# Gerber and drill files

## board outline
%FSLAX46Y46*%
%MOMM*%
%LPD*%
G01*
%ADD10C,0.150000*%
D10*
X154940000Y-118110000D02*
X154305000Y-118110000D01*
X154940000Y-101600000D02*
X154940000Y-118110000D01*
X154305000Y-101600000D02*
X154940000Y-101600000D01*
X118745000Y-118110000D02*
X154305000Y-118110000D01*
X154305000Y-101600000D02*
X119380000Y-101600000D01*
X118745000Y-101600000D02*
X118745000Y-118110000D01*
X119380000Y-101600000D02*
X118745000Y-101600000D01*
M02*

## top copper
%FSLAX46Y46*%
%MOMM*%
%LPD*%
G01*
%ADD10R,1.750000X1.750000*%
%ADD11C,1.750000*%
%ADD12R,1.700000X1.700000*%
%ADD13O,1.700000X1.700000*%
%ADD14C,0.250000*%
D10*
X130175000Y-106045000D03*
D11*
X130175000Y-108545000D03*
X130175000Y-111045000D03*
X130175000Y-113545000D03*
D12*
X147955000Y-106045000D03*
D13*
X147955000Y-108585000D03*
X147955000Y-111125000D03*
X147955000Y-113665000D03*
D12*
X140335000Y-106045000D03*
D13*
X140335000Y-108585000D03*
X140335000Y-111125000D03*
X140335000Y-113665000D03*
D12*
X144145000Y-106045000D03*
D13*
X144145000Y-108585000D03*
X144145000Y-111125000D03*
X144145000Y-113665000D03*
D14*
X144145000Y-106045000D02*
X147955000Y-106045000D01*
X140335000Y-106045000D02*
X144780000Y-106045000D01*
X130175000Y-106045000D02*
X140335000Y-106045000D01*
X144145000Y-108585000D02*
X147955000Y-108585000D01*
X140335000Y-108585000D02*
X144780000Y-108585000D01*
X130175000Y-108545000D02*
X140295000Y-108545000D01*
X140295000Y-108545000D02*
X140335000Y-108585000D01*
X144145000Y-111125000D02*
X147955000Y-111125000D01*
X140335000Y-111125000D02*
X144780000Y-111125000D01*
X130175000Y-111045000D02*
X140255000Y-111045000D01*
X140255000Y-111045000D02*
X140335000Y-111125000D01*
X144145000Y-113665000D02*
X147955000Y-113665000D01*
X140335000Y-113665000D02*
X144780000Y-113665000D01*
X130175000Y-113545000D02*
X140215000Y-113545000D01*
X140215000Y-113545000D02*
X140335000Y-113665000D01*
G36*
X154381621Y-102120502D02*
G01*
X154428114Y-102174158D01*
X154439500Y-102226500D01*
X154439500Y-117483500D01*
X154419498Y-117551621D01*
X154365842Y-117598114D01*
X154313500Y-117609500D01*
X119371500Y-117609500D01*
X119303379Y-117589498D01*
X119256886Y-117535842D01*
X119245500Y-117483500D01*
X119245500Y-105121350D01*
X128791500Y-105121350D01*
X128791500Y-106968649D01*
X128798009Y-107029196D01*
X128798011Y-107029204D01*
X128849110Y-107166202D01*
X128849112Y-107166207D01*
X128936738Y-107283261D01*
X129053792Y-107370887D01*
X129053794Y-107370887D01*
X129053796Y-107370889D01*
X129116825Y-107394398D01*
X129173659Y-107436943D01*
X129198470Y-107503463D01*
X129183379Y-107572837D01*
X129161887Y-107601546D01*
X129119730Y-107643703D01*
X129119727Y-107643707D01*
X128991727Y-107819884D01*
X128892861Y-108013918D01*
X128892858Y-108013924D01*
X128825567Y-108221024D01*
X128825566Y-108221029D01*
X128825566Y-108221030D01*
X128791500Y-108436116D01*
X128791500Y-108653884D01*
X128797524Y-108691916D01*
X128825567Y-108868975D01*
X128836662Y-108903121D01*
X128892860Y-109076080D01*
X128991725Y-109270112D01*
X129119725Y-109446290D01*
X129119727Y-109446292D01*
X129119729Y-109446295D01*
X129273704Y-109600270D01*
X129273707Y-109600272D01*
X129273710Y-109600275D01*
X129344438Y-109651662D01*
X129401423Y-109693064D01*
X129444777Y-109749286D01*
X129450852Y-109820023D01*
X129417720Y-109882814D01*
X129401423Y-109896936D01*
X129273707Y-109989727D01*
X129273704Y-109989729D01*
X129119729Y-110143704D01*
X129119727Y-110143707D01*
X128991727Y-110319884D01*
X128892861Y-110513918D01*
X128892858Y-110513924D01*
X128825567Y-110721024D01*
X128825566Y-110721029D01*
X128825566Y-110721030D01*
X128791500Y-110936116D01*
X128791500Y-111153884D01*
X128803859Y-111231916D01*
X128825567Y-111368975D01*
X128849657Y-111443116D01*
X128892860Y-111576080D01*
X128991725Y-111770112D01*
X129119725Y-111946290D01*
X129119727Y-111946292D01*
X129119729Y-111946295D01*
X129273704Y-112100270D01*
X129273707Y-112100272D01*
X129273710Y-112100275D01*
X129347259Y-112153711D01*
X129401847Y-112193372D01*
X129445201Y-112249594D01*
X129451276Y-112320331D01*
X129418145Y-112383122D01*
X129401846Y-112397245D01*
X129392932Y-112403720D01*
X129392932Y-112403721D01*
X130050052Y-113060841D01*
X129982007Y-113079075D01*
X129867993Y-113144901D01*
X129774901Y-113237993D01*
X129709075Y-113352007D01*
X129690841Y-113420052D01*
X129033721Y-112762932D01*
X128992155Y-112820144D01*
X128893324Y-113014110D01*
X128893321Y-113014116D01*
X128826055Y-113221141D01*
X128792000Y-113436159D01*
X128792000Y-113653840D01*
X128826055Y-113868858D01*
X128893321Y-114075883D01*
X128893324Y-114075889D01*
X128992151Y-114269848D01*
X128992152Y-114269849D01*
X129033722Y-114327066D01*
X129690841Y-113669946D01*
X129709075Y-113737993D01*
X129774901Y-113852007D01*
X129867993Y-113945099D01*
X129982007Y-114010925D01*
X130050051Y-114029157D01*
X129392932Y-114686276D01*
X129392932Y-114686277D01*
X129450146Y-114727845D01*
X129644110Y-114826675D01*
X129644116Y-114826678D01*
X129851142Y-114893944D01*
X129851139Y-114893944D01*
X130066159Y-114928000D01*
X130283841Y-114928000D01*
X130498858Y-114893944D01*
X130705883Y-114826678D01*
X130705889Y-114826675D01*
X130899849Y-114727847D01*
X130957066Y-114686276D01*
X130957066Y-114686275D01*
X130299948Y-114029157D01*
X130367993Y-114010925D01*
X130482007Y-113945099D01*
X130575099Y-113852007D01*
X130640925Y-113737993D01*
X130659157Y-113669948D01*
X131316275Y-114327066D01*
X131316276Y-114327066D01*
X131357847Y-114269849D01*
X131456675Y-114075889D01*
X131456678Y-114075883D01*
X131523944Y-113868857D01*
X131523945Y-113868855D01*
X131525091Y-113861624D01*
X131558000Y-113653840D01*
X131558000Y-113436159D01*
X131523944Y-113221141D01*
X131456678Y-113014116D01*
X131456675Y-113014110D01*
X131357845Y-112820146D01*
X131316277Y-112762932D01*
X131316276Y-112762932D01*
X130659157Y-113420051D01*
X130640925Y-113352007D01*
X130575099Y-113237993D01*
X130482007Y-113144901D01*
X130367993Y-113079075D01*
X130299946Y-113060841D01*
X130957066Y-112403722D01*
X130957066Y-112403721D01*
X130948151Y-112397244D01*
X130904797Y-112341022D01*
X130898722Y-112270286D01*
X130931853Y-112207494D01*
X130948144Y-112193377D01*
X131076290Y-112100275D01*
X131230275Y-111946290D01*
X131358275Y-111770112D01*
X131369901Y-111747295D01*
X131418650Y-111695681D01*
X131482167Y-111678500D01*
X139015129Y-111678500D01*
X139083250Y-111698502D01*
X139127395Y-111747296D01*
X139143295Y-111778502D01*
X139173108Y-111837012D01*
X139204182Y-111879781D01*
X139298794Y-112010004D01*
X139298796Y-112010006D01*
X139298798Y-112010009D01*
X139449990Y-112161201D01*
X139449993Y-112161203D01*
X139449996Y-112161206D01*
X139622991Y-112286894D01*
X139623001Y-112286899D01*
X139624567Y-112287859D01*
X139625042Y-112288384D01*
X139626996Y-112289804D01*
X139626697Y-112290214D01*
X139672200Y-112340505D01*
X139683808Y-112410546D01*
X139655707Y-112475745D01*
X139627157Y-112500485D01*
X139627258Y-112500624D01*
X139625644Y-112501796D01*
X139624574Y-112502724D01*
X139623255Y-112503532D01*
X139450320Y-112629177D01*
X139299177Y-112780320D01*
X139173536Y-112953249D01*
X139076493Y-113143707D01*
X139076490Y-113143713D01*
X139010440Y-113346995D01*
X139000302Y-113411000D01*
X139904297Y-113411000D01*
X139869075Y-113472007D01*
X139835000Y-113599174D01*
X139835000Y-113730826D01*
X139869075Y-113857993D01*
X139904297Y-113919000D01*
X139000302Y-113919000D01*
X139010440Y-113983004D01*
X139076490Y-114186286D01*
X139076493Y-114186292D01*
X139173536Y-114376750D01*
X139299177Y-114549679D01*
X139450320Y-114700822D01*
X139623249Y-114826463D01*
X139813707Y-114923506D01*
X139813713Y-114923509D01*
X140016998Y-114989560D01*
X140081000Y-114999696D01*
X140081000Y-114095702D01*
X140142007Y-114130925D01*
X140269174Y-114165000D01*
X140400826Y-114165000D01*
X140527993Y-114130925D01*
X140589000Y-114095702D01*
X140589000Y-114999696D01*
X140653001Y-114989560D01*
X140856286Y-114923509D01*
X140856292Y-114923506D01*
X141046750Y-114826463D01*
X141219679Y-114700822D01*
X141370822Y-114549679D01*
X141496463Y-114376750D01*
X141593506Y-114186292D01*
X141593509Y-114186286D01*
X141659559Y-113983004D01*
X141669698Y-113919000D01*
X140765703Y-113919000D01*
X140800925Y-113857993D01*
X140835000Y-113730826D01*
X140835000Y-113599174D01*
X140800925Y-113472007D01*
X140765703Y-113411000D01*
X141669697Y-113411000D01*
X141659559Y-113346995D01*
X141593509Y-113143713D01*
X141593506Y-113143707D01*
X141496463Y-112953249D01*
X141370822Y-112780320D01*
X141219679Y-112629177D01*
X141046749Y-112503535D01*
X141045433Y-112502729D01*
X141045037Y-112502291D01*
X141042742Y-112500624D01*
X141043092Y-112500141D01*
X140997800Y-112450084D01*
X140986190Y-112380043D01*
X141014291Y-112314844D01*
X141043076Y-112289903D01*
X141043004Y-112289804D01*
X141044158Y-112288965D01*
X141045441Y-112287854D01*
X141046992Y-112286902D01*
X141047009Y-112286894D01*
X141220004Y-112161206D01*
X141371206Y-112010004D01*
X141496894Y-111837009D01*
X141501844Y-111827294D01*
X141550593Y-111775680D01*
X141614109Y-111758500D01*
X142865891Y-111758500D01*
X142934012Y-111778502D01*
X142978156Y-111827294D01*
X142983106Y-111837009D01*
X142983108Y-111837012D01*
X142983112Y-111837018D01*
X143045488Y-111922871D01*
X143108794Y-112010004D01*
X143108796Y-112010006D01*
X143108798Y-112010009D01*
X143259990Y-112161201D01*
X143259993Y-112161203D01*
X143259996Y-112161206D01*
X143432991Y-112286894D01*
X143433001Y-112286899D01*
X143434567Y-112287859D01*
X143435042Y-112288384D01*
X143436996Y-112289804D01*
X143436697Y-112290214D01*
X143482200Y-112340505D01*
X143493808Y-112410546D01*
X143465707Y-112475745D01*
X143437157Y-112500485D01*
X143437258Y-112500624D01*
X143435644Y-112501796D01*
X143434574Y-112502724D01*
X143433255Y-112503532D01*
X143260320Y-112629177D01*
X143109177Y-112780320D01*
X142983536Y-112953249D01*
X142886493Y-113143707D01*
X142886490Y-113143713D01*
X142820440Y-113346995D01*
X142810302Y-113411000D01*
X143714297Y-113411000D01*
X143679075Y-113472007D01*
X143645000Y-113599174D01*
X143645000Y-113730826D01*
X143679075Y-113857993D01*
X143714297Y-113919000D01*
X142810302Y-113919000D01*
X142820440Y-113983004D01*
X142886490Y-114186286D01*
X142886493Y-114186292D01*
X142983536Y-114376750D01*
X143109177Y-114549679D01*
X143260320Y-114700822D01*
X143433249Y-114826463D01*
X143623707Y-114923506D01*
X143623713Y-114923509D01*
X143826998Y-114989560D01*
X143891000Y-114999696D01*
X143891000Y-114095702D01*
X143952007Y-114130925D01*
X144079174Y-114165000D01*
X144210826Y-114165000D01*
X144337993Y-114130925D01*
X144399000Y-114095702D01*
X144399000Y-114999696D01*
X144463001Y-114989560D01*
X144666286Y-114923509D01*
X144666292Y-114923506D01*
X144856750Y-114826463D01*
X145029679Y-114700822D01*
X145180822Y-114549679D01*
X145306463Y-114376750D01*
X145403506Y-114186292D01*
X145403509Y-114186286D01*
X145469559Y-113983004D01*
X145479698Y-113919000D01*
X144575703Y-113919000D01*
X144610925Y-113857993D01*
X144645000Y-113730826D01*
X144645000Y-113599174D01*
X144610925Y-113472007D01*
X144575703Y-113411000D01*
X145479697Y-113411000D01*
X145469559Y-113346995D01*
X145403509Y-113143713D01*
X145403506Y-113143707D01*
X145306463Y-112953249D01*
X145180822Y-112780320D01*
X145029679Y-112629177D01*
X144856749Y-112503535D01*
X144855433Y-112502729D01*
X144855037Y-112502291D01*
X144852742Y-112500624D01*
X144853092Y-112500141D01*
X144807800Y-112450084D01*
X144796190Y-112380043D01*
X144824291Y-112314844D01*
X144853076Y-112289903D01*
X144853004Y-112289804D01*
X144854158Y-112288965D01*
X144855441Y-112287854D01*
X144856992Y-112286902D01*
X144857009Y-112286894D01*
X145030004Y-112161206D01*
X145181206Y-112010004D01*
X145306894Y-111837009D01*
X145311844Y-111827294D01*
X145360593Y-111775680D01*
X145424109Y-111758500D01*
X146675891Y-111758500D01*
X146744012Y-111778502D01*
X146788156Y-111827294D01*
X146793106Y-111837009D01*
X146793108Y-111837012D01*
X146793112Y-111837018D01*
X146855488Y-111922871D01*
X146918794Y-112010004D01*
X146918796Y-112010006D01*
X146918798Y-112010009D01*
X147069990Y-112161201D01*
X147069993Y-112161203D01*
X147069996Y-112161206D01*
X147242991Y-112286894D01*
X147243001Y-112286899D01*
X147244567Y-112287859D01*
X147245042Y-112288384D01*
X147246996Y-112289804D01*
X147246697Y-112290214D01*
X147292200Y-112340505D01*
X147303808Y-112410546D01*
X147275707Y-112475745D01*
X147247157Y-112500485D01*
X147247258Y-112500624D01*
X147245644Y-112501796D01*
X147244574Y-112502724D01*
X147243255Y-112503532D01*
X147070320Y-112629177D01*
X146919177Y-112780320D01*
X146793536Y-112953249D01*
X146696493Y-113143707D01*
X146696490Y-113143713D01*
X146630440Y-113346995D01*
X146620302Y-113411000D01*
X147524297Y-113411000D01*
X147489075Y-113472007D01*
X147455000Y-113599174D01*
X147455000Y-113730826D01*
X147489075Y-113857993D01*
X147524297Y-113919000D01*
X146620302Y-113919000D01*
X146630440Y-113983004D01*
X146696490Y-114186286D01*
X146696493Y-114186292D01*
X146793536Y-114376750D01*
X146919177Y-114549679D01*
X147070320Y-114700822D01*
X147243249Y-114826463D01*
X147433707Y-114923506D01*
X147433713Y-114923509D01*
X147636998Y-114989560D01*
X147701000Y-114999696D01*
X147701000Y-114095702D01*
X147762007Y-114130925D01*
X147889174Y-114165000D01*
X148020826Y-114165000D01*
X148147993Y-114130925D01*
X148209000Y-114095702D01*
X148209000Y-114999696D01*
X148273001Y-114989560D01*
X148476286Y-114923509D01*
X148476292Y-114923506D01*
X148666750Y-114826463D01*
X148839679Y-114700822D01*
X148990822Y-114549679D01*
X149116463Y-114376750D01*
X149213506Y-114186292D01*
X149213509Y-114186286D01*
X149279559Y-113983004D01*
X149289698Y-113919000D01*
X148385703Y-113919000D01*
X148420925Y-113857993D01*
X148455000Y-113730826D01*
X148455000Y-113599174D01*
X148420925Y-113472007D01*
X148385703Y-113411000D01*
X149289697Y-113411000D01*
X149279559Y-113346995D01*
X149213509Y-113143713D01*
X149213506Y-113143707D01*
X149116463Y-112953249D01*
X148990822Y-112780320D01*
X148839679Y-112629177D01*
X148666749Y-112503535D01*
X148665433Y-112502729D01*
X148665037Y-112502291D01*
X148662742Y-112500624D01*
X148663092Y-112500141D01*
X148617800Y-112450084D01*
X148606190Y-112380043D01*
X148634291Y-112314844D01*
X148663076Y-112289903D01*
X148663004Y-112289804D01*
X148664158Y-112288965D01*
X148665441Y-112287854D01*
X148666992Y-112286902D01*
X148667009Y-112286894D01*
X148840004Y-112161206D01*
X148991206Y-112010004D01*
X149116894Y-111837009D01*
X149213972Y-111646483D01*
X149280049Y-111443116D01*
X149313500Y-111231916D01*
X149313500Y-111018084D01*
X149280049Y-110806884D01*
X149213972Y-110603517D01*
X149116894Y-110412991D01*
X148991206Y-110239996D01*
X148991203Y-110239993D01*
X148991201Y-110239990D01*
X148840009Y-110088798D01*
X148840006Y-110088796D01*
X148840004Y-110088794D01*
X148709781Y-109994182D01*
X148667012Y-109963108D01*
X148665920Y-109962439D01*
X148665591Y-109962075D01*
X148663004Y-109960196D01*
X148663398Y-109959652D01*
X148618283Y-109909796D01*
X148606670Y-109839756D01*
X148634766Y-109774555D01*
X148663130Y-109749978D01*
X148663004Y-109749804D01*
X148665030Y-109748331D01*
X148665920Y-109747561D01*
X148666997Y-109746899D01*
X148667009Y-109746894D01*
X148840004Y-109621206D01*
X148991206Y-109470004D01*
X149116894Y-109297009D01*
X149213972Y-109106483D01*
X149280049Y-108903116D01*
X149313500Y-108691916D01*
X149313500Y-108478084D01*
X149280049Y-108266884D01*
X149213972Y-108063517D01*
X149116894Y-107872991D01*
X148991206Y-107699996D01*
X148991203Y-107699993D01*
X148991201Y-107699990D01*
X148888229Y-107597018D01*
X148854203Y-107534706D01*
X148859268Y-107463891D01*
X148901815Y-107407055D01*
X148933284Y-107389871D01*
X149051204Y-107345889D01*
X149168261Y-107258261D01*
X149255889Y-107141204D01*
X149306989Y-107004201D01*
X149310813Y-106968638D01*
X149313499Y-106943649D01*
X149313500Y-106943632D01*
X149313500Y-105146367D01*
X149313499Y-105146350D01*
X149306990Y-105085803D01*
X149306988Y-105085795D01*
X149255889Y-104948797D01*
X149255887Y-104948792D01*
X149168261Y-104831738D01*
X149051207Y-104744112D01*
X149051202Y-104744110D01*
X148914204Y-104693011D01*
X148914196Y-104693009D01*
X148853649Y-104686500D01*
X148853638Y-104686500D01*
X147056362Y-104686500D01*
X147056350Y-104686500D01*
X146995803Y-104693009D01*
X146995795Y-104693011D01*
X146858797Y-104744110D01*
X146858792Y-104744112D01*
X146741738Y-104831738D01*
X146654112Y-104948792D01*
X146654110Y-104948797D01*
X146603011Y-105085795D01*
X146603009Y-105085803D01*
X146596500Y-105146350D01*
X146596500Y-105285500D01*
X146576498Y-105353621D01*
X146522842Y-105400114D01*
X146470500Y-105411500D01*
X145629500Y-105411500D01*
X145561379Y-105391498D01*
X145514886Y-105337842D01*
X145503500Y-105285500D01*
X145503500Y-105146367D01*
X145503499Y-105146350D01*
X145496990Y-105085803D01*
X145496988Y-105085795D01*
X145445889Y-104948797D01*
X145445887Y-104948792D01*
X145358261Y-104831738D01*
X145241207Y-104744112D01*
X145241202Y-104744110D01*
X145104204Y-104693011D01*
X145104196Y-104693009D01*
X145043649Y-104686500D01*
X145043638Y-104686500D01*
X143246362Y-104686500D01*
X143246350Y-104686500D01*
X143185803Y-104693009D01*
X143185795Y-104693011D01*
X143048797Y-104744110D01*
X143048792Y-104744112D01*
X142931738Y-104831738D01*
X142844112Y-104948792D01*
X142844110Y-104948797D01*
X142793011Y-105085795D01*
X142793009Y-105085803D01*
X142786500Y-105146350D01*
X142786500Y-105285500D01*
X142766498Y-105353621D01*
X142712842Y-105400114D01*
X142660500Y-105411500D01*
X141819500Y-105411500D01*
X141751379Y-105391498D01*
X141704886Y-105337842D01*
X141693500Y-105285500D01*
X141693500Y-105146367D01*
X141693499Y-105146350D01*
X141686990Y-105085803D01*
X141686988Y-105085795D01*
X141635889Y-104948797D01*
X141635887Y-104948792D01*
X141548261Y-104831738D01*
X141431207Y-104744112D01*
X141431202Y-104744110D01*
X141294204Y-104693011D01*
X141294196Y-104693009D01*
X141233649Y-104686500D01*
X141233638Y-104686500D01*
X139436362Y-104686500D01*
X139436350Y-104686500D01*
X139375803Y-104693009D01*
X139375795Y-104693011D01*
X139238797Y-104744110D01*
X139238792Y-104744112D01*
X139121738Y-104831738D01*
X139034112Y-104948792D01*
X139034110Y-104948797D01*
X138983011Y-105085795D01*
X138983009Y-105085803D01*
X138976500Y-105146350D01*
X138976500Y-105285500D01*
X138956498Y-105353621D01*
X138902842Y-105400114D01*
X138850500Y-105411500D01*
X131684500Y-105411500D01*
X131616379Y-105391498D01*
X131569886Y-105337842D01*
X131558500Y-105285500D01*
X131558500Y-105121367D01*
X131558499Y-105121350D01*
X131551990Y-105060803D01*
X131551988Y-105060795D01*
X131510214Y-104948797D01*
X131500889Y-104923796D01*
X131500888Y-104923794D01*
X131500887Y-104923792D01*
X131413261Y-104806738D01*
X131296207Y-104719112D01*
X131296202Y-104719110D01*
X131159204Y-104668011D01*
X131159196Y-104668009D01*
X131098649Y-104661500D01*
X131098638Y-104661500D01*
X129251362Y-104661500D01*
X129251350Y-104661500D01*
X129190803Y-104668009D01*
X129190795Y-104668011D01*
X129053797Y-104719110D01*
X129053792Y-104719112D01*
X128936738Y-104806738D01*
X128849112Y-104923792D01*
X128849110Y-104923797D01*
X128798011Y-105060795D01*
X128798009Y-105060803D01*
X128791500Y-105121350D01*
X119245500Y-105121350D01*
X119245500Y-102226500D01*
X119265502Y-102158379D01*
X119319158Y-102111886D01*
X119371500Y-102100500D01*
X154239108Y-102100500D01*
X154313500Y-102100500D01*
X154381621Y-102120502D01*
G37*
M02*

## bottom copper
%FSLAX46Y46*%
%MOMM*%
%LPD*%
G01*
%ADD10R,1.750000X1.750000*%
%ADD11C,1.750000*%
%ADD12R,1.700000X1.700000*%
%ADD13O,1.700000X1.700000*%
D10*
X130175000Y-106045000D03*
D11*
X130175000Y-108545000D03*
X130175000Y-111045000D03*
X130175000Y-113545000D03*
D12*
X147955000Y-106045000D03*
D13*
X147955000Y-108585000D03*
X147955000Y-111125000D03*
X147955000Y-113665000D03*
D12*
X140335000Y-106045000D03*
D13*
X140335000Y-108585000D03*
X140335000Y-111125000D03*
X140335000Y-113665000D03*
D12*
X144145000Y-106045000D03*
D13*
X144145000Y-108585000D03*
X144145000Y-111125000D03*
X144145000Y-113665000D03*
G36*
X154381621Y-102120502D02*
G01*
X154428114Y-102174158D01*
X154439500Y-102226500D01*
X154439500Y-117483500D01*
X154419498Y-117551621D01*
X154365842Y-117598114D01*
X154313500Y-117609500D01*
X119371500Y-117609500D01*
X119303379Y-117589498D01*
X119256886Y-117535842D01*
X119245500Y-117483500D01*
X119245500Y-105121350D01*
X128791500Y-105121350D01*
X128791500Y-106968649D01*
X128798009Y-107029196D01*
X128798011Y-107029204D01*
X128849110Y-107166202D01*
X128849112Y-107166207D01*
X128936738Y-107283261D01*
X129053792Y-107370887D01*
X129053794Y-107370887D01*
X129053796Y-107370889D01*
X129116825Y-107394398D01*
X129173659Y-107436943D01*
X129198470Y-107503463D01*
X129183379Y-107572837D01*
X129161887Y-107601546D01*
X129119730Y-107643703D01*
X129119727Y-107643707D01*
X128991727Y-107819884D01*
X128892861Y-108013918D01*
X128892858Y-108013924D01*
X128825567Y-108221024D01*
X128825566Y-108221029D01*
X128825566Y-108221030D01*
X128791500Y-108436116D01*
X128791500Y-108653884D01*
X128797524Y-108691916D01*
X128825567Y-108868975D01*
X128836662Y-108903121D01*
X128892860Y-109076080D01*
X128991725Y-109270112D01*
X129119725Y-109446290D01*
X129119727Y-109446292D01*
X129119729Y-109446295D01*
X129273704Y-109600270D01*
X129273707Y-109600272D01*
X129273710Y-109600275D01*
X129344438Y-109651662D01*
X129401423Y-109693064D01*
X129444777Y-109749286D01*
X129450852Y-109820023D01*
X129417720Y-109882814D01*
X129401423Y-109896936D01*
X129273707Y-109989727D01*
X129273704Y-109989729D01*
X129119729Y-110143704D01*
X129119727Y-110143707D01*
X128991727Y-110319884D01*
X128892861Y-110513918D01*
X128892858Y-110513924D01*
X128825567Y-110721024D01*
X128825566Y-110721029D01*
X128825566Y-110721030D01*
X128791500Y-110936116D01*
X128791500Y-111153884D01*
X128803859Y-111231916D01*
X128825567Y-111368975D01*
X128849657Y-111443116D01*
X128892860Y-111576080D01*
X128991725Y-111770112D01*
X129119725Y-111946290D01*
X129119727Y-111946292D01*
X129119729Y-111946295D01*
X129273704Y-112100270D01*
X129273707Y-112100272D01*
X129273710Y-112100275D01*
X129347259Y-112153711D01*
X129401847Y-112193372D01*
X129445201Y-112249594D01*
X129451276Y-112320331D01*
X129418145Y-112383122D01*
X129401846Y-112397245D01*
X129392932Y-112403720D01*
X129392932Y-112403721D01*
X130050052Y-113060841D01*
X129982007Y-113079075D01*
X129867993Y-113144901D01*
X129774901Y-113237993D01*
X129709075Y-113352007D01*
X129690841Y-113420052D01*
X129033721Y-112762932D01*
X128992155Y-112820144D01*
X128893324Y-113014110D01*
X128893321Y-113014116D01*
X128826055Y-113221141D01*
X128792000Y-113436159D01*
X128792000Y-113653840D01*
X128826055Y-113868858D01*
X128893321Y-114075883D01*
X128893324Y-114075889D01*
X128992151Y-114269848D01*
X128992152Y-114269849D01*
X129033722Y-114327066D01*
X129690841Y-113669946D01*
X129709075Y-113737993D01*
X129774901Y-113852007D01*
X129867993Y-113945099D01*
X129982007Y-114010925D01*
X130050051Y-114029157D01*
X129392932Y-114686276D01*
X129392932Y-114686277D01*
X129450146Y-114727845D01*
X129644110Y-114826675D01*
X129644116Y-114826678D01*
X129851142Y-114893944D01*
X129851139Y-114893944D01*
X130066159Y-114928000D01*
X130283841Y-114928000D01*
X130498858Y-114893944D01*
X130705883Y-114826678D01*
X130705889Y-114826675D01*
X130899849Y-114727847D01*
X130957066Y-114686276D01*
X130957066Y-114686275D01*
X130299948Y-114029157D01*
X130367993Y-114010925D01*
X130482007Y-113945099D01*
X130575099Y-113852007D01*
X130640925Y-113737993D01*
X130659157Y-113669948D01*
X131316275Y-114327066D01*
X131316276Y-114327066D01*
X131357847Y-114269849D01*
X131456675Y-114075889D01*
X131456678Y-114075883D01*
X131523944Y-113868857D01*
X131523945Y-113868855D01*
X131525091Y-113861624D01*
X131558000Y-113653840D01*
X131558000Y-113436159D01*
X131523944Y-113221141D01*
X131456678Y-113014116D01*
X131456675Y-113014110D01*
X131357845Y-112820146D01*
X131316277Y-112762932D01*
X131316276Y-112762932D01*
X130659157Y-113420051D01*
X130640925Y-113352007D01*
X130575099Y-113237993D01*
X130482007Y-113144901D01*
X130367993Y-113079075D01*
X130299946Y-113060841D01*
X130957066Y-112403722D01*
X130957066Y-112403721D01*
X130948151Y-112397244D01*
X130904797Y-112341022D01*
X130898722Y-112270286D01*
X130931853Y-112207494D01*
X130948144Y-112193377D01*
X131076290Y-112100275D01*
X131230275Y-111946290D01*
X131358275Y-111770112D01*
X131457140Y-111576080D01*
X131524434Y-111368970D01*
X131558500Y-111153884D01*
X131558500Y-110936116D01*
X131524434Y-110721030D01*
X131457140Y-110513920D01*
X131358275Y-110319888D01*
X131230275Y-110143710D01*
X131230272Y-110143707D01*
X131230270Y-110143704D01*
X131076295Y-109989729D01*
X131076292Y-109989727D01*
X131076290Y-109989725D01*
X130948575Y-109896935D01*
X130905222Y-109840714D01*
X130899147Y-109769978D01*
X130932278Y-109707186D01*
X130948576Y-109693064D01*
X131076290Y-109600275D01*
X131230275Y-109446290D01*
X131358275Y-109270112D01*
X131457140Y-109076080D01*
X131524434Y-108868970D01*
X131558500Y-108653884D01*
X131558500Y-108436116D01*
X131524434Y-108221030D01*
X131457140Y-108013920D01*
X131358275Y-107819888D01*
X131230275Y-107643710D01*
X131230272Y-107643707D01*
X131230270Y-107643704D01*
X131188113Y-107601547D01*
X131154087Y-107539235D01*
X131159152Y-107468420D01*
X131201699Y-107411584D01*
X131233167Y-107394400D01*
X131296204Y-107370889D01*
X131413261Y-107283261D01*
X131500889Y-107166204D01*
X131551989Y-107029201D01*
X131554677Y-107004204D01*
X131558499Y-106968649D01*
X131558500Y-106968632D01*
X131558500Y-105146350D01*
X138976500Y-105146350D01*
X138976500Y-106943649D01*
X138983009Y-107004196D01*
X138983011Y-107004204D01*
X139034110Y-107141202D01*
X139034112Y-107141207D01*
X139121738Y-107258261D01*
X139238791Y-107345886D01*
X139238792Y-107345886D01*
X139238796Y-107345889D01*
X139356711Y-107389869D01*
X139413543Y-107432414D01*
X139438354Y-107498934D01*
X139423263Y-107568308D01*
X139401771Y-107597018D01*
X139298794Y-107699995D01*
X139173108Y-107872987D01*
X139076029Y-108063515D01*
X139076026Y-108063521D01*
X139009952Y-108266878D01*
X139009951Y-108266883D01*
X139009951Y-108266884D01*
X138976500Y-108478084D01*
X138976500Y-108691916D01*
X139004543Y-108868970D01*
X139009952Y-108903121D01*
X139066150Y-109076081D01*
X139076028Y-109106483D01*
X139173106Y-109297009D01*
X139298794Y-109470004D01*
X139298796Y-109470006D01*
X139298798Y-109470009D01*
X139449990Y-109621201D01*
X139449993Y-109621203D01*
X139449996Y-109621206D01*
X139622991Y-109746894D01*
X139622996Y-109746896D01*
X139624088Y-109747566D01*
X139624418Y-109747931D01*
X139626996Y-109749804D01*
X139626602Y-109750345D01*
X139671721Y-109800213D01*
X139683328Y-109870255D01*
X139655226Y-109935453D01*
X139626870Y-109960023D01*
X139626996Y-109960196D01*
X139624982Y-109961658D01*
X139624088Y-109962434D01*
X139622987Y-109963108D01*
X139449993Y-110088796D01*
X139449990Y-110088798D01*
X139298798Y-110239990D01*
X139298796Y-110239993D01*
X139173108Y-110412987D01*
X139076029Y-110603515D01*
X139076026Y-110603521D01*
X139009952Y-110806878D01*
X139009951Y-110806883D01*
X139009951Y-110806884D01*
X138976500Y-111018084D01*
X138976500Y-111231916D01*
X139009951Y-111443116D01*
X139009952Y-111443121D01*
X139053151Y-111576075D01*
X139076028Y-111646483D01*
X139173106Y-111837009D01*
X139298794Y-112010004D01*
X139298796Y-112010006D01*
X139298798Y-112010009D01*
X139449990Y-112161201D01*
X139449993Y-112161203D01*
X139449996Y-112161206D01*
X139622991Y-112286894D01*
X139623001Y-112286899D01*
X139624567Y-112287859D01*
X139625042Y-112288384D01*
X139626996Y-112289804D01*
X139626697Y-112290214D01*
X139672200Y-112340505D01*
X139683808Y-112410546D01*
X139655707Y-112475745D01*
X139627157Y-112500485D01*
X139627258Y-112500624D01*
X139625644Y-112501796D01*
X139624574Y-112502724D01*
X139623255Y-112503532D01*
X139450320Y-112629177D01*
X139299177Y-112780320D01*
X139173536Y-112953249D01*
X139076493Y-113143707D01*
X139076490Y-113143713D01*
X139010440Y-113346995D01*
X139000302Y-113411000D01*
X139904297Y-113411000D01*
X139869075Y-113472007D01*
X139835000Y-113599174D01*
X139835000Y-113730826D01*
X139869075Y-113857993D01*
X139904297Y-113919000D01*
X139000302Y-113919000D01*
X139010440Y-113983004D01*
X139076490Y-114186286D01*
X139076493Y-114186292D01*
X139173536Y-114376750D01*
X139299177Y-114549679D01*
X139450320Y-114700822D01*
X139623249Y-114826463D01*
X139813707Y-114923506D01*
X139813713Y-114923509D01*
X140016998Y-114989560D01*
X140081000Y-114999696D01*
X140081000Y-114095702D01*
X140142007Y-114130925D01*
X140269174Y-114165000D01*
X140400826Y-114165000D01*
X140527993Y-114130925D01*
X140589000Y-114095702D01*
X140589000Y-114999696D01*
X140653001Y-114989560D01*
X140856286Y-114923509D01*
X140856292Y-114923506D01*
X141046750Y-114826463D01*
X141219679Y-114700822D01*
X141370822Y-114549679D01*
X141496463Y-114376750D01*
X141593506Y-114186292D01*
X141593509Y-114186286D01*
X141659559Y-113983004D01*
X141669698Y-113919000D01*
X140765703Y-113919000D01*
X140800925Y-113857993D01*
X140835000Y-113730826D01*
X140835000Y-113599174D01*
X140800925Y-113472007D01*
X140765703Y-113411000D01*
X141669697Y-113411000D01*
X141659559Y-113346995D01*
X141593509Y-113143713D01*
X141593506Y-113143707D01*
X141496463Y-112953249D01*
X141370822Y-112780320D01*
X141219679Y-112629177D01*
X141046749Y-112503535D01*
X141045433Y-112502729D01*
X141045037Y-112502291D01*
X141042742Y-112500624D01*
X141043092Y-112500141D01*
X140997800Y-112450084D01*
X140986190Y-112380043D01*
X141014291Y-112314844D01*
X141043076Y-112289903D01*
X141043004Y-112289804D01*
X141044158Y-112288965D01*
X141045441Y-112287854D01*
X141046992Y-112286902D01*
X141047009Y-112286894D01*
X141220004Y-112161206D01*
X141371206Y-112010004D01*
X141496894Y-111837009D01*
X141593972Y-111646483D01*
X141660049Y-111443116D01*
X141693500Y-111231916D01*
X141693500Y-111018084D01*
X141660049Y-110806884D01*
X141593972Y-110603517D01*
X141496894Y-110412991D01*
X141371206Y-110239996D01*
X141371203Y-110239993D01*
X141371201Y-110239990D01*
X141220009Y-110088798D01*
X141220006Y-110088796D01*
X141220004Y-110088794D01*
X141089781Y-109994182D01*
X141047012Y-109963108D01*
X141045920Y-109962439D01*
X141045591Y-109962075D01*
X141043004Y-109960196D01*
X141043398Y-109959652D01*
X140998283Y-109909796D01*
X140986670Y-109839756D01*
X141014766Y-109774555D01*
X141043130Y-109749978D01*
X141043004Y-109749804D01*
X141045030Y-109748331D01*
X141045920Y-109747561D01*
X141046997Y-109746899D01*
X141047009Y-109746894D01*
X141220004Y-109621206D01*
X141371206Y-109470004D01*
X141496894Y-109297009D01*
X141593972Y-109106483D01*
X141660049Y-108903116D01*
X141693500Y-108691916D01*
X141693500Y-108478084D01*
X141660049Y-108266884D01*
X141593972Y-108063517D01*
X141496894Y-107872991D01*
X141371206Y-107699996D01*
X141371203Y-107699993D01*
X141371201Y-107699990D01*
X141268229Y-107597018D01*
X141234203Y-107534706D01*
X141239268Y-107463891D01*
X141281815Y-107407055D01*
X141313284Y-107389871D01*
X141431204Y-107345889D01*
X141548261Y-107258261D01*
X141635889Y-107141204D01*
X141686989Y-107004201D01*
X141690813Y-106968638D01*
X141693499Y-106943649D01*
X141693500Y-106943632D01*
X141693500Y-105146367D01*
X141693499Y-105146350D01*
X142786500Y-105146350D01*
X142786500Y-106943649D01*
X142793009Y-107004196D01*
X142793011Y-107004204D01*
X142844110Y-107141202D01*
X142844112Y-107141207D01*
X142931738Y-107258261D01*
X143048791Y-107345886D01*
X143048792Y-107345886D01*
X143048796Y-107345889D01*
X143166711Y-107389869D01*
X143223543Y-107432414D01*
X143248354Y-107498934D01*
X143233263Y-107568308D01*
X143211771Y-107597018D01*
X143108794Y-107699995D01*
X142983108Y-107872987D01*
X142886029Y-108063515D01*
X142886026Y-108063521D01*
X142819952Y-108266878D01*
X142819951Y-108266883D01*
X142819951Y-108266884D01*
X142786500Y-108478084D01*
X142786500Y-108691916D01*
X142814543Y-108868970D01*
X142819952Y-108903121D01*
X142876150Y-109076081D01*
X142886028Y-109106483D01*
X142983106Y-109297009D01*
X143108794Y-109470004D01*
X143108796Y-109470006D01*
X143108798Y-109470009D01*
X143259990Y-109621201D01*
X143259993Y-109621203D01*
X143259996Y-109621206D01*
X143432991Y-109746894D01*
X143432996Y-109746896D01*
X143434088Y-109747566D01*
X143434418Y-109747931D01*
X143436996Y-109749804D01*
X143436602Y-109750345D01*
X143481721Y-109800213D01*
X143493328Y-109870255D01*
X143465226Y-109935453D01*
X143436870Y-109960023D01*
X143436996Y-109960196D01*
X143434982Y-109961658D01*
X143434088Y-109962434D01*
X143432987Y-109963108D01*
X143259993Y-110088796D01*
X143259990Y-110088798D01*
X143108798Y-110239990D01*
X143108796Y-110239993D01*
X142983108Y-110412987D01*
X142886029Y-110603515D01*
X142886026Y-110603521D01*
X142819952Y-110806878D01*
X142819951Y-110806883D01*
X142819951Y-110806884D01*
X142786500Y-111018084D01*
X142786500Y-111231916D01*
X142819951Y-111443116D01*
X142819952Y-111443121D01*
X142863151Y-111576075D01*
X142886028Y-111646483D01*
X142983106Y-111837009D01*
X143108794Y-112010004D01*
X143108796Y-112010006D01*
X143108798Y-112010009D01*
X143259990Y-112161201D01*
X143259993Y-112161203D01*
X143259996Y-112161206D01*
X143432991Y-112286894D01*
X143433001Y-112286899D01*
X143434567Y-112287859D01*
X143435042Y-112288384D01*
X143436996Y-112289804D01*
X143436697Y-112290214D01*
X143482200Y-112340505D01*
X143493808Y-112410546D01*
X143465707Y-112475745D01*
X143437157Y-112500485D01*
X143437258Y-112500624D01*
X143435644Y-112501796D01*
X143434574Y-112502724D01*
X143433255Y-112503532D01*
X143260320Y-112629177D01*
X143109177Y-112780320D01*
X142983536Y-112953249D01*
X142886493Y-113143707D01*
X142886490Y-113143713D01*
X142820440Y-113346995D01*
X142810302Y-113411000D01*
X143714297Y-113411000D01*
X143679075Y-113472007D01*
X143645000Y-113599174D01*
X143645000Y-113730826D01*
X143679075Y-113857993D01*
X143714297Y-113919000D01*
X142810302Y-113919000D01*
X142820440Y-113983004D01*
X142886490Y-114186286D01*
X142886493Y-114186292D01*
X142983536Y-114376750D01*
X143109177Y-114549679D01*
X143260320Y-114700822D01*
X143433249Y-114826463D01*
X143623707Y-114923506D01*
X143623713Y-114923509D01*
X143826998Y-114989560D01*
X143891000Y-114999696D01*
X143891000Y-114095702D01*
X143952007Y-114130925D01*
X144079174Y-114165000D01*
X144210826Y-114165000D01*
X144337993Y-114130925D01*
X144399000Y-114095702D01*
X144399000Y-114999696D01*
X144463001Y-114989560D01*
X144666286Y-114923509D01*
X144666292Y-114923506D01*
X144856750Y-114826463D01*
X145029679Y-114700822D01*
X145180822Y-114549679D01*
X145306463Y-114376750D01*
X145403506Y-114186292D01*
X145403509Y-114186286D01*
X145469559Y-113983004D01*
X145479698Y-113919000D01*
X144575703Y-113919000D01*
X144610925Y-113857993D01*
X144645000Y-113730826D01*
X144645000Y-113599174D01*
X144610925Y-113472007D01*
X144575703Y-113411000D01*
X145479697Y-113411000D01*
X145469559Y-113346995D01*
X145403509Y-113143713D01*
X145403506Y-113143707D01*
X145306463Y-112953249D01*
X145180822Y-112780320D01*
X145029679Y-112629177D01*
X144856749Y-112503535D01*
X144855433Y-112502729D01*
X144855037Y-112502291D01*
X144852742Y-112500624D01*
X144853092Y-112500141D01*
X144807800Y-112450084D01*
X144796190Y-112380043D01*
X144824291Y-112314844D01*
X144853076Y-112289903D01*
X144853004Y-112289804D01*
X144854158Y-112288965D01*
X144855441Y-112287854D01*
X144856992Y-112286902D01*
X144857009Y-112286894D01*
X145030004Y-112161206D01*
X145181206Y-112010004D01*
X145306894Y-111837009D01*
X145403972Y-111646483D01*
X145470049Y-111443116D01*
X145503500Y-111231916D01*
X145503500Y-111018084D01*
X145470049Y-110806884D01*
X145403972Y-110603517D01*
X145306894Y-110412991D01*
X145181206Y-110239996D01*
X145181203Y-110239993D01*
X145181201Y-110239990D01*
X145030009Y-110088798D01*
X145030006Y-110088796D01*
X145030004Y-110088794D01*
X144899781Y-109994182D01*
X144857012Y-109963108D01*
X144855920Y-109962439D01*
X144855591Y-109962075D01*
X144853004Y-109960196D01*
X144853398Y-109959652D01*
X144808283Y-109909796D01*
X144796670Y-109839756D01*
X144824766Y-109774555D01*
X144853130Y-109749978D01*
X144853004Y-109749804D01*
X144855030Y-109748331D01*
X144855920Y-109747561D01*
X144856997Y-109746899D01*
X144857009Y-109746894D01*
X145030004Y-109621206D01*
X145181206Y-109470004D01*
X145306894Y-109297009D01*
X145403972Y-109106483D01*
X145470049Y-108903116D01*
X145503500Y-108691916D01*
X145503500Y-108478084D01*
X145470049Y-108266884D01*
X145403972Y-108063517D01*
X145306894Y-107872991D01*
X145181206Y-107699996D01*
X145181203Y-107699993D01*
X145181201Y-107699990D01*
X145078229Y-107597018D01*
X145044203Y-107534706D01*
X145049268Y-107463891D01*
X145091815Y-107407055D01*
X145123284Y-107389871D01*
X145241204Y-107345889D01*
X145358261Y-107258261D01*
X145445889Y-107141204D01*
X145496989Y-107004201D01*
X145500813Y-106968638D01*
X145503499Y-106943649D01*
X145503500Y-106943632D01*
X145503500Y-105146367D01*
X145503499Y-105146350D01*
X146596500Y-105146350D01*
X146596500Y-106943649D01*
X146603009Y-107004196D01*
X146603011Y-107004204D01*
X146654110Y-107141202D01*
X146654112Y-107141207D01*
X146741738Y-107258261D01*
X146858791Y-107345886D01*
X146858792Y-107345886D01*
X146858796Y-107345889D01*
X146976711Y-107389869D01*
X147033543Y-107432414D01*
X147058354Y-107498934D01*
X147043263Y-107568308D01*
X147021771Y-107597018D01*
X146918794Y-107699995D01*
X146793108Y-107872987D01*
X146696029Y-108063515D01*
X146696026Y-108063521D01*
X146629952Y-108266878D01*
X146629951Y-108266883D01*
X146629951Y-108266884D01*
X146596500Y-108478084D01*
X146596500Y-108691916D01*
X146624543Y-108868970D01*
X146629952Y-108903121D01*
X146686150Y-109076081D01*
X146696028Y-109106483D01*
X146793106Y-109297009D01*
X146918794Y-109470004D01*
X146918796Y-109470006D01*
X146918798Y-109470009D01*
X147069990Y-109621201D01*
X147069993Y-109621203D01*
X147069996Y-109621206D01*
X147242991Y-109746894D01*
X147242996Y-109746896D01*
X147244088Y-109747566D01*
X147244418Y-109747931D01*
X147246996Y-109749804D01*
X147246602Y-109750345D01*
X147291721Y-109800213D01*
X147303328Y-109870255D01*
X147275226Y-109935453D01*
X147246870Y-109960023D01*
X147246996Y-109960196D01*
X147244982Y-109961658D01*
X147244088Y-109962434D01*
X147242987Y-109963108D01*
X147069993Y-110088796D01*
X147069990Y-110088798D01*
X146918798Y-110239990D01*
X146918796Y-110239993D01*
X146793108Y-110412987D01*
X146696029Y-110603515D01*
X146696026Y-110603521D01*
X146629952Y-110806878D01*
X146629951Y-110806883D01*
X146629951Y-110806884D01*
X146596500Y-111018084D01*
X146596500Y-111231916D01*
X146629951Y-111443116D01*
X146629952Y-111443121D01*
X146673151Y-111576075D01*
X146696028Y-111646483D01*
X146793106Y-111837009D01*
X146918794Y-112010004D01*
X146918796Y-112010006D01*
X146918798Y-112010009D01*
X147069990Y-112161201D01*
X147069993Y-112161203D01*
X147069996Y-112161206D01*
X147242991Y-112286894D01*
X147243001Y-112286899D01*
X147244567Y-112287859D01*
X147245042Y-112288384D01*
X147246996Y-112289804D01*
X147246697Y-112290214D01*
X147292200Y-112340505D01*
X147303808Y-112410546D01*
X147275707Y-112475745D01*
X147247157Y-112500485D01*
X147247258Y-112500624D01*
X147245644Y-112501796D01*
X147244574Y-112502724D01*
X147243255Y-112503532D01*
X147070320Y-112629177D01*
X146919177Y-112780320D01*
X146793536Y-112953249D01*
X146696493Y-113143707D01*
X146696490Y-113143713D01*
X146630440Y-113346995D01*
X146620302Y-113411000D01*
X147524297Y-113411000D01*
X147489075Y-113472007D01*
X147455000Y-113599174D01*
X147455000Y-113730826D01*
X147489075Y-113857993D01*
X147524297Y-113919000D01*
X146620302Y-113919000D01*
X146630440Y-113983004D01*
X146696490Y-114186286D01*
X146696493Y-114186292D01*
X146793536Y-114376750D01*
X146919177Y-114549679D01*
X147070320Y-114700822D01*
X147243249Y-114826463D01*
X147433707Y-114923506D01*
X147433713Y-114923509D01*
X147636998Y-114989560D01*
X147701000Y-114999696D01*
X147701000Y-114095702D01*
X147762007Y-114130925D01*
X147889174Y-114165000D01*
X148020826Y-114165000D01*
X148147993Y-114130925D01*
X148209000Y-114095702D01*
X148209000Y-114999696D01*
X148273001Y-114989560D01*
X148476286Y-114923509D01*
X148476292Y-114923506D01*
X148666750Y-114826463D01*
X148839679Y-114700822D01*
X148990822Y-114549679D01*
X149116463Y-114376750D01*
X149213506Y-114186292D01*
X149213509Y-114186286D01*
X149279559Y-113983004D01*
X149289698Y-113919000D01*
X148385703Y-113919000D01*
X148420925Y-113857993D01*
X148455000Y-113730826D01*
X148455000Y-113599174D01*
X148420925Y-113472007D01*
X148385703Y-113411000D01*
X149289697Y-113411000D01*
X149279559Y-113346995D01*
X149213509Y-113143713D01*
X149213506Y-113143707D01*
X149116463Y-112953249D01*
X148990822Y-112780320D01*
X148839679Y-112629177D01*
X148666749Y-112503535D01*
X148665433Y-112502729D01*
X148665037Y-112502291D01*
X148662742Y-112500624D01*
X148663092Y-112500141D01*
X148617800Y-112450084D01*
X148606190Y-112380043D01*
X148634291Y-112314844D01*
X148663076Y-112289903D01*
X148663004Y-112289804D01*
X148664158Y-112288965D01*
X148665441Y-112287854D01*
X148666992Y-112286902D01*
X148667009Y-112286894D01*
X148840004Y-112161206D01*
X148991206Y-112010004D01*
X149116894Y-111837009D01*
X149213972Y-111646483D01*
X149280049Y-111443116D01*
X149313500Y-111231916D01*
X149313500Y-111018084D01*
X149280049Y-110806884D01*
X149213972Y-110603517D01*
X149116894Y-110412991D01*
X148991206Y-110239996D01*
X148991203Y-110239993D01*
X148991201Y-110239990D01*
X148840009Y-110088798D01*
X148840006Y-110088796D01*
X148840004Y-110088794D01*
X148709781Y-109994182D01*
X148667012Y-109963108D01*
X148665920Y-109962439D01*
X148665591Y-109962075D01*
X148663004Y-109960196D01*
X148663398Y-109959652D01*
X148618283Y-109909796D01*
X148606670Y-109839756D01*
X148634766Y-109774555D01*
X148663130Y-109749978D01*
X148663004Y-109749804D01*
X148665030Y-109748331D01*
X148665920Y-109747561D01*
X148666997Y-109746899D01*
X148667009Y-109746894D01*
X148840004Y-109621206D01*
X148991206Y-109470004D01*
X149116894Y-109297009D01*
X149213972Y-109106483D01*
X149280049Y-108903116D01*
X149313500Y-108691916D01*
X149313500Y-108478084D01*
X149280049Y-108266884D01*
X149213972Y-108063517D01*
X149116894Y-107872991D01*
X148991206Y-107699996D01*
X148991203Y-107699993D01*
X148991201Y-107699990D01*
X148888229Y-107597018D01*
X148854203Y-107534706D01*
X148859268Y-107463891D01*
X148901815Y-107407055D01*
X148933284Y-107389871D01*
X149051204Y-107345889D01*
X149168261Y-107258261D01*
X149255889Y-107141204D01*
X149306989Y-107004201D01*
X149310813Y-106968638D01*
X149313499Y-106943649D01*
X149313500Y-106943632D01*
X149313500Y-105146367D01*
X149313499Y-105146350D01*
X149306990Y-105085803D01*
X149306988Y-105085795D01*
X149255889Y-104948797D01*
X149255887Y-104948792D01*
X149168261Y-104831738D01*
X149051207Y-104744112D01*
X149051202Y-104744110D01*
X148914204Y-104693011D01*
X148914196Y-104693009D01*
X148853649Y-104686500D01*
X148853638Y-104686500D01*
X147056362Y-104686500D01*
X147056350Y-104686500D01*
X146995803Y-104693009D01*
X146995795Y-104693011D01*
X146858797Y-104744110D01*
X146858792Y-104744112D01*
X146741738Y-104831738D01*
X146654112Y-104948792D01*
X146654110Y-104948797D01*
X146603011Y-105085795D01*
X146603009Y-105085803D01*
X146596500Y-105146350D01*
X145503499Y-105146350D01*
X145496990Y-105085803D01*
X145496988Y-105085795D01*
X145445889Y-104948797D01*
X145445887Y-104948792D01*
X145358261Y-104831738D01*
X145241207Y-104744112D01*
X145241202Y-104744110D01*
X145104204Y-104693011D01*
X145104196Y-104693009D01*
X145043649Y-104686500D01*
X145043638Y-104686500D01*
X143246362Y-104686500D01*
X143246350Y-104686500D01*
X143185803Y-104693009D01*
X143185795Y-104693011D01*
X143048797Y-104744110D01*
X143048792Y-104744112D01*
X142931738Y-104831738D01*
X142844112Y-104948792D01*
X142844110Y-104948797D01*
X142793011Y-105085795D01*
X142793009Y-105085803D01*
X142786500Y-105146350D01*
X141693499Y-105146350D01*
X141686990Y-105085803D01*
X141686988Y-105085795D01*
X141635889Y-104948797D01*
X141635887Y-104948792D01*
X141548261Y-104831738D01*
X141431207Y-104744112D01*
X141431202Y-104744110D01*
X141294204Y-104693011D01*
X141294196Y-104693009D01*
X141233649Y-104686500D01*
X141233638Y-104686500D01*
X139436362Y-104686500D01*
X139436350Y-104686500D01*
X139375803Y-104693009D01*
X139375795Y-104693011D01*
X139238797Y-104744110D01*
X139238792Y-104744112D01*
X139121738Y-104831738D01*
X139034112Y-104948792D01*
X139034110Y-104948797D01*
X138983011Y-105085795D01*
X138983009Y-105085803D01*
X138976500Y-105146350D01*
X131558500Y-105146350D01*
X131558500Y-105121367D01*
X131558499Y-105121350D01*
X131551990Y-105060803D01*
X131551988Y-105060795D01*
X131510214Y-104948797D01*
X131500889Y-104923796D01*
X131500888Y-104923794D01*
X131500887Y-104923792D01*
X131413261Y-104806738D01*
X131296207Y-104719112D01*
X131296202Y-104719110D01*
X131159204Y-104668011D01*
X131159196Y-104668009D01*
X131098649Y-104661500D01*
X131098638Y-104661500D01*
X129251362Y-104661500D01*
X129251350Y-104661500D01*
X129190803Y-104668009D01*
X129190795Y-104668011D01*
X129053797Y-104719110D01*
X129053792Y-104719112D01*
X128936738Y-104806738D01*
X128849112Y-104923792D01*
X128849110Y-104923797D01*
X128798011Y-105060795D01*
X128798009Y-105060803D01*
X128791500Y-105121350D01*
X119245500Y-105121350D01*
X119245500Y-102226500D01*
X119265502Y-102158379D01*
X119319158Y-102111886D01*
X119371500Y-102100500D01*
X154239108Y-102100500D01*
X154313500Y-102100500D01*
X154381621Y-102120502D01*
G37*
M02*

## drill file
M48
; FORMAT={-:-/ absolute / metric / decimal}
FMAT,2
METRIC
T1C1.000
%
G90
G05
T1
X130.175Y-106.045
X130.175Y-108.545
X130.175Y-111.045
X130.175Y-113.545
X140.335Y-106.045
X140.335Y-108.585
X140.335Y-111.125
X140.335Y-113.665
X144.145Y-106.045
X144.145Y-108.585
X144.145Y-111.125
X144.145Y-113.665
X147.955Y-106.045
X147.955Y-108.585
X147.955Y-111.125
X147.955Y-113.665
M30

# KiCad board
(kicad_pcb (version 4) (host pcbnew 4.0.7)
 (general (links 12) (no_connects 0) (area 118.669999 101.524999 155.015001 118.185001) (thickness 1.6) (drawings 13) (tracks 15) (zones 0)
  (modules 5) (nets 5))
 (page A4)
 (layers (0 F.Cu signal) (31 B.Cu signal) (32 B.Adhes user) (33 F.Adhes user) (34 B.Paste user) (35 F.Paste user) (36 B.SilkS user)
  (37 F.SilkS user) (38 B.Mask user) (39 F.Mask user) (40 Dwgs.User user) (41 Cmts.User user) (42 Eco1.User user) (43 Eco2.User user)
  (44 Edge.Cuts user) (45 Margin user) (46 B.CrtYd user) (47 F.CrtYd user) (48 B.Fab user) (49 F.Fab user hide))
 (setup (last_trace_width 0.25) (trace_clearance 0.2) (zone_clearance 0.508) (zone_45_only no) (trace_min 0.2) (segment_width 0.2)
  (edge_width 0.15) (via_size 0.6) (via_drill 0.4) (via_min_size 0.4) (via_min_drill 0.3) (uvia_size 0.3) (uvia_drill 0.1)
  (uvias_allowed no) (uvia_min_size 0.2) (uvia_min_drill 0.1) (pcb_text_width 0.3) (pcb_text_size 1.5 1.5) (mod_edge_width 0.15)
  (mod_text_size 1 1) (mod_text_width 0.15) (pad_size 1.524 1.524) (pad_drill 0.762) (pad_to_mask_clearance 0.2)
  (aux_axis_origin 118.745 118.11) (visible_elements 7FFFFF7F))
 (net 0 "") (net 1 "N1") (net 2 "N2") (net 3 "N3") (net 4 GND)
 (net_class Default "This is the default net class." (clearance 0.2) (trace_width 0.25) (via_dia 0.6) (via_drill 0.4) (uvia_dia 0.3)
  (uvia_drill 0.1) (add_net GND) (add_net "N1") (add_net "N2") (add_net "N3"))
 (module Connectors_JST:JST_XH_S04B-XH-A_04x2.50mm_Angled (layer F.Cu) (at 130.175 106.045 270)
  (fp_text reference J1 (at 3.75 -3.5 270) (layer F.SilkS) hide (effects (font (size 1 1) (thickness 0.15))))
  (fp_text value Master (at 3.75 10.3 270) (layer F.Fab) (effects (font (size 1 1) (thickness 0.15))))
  (pad 1 thru_hole rect (at 0 0 270) (size 1.75 1.75) (drill 1) (layers *.Cu *.Mask F.SilkS) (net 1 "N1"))
  (pad 2 thru_hole circle (at 2.5 0 270) (size 1.75 1.75) (drill 1) (layers *.Cu *.Mask F.SilkS) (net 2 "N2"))
  (pad 3 thru_hole circle (at 5 0 270) (size 1.75 1.75) (drill 1) (layers *.Cu *.Mask F.SilkS) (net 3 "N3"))
  (pad 4 thru_hole circle (at 7.5 0 270) (size 1.75 1.75) (drill 1) (layers *.Cu *.Mask F.SilkS) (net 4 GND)))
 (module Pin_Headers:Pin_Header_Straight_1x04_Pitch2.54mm (layer F.Cu) (at 147.955 106.045)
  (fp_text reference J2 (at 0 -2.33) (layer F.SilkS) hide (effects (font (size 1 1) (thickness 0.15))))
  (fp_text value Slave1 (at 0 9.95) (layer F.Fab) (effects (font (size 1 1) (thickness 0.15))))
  (pad 1 thru_hole rect (at 0 0) (size 1.7 1.7) (drill 1) (layers *.Cu *.Mask) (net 1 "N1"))
  (pad 2 thru_hole oval (at 0 2.54) (size 1.7 1.7) (drill 1) (layers *.Cu *.Mask) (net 2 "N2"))
  (pad 3 thru_hole oval (at 0 5.08) (size 1.7 1.7) (drill 1) (layers *.Cu *.Mask) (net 3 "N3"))
  (pad 4 thru_hole oval (at 0 7.62) (size 1.7 1.7) (drill 1) (layers *.Cu *.Mask) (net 4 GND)))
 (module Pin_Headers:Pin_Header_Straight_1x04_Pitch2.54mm (layer F.Cu) (at 140.335 106.045)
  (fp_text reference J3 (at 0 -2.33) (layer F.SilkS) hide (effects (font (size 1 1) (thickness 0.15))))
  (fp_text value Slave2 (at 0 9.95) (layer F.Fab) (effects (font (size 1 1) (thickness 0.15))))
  (pad 1 thru_hole rect (at 0 0) (size 1.7 1.7) (drill 1) (layers *.Cu *.Mask) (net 1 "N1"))
  (pad 2 thru_hole oval (at 0 2.54) (size 1.7 1.7) (drill 1) (layers *.Cu *.Mask) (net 2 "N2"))
  (pad 3 thru_hole oval (at 0 5.08) (size 1.7 1.7) (drill 1) (layers *.Cu *.Mask) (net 3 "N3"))
  (pad 4 thru_hole oval (at 0 7.62) (size 1.7 1.7) (drill 1) (layers *.Cu *.Mask) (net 4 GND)))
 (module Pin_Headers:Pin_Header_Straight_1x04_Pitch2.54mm (layer F.Cu) (at 144.145 106.045)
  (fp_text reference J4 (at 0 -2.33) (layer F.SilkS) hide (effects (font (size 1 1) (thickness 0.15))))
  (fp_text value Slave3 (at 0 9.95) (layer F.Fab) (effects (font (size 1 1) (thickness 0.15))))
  (pad 1 thru_hole rect (at 0 0) (size 1.7 1.7) (drill 1) (layers *.Cu *.Mask) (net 1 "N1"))
  (pad 2 thru_hole oval (at 0 2.54) (size 1.7 1.7) (drill 1) (layers *.Cu *.Mask) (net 2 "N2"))
  (pad 3 thru_hole oval (at 0 5.08) (size 1.7 1.7) (drill 1) (layers *.Cu *.Mask) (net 3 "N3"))
  (pad 4 thru_hole oval (at 0 7.62) (size 1.7 1.7) (drill 1) (layers *.Cu *.Mask) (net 4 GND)))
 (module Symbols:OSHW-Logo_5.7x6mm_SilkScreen (layer B.Cu) (at 135.255 109.855 270)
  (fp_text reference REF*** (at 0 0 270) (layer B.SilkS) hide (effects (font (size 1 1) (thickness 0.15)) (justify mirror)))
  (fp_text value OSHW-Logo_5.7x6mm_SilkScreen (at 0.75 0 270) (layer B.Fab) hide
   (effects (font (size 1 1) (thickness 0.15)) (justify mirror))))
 (gr_line (start 154.94 118.11) (end 154.305 118.11) (layer Edge.Cuts) (width 0.15))
 (gr_line (start 154.94 101.6) (end 154.94 118.11) (layer Edge.Cuts) (width 0.15))
 (gr_line (start 154.305 101.6) (end 154.94 101.6) (layer Edge.Cuts) (width 0.15))
 (gr_line (start 118.745 118.11) (end 154.305 118.11) (layer Edge.Cuts) (width 0.15))
 (gr_line (start 154.305 101.6) (end 119.38 101.6) (layer Edge.Cuts) (width 0.15))
 (gr_line (start 118.745 101.6) (end 118.745 118.11) (layer Edge.Cuts) (width 0.15))
 (gr_line (start 119.38 101.6) (end 118.745 101.6) (layer Edge.Cuts) (width 0.15))
 (segment (start 144.145 106.045) (end 147.955 106.045) (width 0.25) (layer F.Cu) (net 1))
 (segment (start 140.335 106.045) (end 144.78 106.045) (width 0.25) (layer F.Cu) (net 1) (status 30))
 (segment (start 130.175 106.045) (end 140.335 106.045) (width 0.25) (layer F.Cu) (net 1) (status 30))
 (segment (start 144.145 108.585) (end 147.955 108.585) (width 0.25) (layer F.Cu) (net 2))
 (segment (start 140.335 108.585) (end 144.78 108.585) (width 0.25) (layer F.Cu) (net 2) (status 30))
 (segment (start 130.175 108.545) (end 140.295 108.545) (width 0.25) (layer F.Cu) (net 2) (status 30))
 (segment (start 140.295 108.545) (end 140.335 108.585) (width 0.25) (layer F.Cu) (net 2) (status 30))
 (segment (start 144.145 111.125) (end 147.955 111.125) (width 0.25) (layer F.Cu) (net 3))
 (segment (start 140.335 111.125) (end 144.78 111.125) (width 0.25) (layer F.Cu) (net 3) (status 30))
 (segment (start 130.175 111.045) (end 140.255 111.045) (width 0.25) (layer F.Cu) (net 3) (status 30))
 (segment (start 140.255 111.045) (end 140.335 111.125) (width 0.25) (layer F.Cu) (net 3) (status 30))
 (segment (start 144.145 113.665) (end 147.955 113.665) (width 0.25) (layer F.Cu) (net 4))
 (segment (start 140.335 113.665) (end 144.78 113.665) (width 0.25) (layer F.Cu) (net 4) (status 30))
 (segment (start 130.175 113.545) (end 140.215 113.545) (width 0.25) (layer F.Cu) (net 4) (status 30))
 (segment (start 140.215 113.545) (end 140.335 113.665) (width 0.25) (layer F.Cu) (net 4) (status 30))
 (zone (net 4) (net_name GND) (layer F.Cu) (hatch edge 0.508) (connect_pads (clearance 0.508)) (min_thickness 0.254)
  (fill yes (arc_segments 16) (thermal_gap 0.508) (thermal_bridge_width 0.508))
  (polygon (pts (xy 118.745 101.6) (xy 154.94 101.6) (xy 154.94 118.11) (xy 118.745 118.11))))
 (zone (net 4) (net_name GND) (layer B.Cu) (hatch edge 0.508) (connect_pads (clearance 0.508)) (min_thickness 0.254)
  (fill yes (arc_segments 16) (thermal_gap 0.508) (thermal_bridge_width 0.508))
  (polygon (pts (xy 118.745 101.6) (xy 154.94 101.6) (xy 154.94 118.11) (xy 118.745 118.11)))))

